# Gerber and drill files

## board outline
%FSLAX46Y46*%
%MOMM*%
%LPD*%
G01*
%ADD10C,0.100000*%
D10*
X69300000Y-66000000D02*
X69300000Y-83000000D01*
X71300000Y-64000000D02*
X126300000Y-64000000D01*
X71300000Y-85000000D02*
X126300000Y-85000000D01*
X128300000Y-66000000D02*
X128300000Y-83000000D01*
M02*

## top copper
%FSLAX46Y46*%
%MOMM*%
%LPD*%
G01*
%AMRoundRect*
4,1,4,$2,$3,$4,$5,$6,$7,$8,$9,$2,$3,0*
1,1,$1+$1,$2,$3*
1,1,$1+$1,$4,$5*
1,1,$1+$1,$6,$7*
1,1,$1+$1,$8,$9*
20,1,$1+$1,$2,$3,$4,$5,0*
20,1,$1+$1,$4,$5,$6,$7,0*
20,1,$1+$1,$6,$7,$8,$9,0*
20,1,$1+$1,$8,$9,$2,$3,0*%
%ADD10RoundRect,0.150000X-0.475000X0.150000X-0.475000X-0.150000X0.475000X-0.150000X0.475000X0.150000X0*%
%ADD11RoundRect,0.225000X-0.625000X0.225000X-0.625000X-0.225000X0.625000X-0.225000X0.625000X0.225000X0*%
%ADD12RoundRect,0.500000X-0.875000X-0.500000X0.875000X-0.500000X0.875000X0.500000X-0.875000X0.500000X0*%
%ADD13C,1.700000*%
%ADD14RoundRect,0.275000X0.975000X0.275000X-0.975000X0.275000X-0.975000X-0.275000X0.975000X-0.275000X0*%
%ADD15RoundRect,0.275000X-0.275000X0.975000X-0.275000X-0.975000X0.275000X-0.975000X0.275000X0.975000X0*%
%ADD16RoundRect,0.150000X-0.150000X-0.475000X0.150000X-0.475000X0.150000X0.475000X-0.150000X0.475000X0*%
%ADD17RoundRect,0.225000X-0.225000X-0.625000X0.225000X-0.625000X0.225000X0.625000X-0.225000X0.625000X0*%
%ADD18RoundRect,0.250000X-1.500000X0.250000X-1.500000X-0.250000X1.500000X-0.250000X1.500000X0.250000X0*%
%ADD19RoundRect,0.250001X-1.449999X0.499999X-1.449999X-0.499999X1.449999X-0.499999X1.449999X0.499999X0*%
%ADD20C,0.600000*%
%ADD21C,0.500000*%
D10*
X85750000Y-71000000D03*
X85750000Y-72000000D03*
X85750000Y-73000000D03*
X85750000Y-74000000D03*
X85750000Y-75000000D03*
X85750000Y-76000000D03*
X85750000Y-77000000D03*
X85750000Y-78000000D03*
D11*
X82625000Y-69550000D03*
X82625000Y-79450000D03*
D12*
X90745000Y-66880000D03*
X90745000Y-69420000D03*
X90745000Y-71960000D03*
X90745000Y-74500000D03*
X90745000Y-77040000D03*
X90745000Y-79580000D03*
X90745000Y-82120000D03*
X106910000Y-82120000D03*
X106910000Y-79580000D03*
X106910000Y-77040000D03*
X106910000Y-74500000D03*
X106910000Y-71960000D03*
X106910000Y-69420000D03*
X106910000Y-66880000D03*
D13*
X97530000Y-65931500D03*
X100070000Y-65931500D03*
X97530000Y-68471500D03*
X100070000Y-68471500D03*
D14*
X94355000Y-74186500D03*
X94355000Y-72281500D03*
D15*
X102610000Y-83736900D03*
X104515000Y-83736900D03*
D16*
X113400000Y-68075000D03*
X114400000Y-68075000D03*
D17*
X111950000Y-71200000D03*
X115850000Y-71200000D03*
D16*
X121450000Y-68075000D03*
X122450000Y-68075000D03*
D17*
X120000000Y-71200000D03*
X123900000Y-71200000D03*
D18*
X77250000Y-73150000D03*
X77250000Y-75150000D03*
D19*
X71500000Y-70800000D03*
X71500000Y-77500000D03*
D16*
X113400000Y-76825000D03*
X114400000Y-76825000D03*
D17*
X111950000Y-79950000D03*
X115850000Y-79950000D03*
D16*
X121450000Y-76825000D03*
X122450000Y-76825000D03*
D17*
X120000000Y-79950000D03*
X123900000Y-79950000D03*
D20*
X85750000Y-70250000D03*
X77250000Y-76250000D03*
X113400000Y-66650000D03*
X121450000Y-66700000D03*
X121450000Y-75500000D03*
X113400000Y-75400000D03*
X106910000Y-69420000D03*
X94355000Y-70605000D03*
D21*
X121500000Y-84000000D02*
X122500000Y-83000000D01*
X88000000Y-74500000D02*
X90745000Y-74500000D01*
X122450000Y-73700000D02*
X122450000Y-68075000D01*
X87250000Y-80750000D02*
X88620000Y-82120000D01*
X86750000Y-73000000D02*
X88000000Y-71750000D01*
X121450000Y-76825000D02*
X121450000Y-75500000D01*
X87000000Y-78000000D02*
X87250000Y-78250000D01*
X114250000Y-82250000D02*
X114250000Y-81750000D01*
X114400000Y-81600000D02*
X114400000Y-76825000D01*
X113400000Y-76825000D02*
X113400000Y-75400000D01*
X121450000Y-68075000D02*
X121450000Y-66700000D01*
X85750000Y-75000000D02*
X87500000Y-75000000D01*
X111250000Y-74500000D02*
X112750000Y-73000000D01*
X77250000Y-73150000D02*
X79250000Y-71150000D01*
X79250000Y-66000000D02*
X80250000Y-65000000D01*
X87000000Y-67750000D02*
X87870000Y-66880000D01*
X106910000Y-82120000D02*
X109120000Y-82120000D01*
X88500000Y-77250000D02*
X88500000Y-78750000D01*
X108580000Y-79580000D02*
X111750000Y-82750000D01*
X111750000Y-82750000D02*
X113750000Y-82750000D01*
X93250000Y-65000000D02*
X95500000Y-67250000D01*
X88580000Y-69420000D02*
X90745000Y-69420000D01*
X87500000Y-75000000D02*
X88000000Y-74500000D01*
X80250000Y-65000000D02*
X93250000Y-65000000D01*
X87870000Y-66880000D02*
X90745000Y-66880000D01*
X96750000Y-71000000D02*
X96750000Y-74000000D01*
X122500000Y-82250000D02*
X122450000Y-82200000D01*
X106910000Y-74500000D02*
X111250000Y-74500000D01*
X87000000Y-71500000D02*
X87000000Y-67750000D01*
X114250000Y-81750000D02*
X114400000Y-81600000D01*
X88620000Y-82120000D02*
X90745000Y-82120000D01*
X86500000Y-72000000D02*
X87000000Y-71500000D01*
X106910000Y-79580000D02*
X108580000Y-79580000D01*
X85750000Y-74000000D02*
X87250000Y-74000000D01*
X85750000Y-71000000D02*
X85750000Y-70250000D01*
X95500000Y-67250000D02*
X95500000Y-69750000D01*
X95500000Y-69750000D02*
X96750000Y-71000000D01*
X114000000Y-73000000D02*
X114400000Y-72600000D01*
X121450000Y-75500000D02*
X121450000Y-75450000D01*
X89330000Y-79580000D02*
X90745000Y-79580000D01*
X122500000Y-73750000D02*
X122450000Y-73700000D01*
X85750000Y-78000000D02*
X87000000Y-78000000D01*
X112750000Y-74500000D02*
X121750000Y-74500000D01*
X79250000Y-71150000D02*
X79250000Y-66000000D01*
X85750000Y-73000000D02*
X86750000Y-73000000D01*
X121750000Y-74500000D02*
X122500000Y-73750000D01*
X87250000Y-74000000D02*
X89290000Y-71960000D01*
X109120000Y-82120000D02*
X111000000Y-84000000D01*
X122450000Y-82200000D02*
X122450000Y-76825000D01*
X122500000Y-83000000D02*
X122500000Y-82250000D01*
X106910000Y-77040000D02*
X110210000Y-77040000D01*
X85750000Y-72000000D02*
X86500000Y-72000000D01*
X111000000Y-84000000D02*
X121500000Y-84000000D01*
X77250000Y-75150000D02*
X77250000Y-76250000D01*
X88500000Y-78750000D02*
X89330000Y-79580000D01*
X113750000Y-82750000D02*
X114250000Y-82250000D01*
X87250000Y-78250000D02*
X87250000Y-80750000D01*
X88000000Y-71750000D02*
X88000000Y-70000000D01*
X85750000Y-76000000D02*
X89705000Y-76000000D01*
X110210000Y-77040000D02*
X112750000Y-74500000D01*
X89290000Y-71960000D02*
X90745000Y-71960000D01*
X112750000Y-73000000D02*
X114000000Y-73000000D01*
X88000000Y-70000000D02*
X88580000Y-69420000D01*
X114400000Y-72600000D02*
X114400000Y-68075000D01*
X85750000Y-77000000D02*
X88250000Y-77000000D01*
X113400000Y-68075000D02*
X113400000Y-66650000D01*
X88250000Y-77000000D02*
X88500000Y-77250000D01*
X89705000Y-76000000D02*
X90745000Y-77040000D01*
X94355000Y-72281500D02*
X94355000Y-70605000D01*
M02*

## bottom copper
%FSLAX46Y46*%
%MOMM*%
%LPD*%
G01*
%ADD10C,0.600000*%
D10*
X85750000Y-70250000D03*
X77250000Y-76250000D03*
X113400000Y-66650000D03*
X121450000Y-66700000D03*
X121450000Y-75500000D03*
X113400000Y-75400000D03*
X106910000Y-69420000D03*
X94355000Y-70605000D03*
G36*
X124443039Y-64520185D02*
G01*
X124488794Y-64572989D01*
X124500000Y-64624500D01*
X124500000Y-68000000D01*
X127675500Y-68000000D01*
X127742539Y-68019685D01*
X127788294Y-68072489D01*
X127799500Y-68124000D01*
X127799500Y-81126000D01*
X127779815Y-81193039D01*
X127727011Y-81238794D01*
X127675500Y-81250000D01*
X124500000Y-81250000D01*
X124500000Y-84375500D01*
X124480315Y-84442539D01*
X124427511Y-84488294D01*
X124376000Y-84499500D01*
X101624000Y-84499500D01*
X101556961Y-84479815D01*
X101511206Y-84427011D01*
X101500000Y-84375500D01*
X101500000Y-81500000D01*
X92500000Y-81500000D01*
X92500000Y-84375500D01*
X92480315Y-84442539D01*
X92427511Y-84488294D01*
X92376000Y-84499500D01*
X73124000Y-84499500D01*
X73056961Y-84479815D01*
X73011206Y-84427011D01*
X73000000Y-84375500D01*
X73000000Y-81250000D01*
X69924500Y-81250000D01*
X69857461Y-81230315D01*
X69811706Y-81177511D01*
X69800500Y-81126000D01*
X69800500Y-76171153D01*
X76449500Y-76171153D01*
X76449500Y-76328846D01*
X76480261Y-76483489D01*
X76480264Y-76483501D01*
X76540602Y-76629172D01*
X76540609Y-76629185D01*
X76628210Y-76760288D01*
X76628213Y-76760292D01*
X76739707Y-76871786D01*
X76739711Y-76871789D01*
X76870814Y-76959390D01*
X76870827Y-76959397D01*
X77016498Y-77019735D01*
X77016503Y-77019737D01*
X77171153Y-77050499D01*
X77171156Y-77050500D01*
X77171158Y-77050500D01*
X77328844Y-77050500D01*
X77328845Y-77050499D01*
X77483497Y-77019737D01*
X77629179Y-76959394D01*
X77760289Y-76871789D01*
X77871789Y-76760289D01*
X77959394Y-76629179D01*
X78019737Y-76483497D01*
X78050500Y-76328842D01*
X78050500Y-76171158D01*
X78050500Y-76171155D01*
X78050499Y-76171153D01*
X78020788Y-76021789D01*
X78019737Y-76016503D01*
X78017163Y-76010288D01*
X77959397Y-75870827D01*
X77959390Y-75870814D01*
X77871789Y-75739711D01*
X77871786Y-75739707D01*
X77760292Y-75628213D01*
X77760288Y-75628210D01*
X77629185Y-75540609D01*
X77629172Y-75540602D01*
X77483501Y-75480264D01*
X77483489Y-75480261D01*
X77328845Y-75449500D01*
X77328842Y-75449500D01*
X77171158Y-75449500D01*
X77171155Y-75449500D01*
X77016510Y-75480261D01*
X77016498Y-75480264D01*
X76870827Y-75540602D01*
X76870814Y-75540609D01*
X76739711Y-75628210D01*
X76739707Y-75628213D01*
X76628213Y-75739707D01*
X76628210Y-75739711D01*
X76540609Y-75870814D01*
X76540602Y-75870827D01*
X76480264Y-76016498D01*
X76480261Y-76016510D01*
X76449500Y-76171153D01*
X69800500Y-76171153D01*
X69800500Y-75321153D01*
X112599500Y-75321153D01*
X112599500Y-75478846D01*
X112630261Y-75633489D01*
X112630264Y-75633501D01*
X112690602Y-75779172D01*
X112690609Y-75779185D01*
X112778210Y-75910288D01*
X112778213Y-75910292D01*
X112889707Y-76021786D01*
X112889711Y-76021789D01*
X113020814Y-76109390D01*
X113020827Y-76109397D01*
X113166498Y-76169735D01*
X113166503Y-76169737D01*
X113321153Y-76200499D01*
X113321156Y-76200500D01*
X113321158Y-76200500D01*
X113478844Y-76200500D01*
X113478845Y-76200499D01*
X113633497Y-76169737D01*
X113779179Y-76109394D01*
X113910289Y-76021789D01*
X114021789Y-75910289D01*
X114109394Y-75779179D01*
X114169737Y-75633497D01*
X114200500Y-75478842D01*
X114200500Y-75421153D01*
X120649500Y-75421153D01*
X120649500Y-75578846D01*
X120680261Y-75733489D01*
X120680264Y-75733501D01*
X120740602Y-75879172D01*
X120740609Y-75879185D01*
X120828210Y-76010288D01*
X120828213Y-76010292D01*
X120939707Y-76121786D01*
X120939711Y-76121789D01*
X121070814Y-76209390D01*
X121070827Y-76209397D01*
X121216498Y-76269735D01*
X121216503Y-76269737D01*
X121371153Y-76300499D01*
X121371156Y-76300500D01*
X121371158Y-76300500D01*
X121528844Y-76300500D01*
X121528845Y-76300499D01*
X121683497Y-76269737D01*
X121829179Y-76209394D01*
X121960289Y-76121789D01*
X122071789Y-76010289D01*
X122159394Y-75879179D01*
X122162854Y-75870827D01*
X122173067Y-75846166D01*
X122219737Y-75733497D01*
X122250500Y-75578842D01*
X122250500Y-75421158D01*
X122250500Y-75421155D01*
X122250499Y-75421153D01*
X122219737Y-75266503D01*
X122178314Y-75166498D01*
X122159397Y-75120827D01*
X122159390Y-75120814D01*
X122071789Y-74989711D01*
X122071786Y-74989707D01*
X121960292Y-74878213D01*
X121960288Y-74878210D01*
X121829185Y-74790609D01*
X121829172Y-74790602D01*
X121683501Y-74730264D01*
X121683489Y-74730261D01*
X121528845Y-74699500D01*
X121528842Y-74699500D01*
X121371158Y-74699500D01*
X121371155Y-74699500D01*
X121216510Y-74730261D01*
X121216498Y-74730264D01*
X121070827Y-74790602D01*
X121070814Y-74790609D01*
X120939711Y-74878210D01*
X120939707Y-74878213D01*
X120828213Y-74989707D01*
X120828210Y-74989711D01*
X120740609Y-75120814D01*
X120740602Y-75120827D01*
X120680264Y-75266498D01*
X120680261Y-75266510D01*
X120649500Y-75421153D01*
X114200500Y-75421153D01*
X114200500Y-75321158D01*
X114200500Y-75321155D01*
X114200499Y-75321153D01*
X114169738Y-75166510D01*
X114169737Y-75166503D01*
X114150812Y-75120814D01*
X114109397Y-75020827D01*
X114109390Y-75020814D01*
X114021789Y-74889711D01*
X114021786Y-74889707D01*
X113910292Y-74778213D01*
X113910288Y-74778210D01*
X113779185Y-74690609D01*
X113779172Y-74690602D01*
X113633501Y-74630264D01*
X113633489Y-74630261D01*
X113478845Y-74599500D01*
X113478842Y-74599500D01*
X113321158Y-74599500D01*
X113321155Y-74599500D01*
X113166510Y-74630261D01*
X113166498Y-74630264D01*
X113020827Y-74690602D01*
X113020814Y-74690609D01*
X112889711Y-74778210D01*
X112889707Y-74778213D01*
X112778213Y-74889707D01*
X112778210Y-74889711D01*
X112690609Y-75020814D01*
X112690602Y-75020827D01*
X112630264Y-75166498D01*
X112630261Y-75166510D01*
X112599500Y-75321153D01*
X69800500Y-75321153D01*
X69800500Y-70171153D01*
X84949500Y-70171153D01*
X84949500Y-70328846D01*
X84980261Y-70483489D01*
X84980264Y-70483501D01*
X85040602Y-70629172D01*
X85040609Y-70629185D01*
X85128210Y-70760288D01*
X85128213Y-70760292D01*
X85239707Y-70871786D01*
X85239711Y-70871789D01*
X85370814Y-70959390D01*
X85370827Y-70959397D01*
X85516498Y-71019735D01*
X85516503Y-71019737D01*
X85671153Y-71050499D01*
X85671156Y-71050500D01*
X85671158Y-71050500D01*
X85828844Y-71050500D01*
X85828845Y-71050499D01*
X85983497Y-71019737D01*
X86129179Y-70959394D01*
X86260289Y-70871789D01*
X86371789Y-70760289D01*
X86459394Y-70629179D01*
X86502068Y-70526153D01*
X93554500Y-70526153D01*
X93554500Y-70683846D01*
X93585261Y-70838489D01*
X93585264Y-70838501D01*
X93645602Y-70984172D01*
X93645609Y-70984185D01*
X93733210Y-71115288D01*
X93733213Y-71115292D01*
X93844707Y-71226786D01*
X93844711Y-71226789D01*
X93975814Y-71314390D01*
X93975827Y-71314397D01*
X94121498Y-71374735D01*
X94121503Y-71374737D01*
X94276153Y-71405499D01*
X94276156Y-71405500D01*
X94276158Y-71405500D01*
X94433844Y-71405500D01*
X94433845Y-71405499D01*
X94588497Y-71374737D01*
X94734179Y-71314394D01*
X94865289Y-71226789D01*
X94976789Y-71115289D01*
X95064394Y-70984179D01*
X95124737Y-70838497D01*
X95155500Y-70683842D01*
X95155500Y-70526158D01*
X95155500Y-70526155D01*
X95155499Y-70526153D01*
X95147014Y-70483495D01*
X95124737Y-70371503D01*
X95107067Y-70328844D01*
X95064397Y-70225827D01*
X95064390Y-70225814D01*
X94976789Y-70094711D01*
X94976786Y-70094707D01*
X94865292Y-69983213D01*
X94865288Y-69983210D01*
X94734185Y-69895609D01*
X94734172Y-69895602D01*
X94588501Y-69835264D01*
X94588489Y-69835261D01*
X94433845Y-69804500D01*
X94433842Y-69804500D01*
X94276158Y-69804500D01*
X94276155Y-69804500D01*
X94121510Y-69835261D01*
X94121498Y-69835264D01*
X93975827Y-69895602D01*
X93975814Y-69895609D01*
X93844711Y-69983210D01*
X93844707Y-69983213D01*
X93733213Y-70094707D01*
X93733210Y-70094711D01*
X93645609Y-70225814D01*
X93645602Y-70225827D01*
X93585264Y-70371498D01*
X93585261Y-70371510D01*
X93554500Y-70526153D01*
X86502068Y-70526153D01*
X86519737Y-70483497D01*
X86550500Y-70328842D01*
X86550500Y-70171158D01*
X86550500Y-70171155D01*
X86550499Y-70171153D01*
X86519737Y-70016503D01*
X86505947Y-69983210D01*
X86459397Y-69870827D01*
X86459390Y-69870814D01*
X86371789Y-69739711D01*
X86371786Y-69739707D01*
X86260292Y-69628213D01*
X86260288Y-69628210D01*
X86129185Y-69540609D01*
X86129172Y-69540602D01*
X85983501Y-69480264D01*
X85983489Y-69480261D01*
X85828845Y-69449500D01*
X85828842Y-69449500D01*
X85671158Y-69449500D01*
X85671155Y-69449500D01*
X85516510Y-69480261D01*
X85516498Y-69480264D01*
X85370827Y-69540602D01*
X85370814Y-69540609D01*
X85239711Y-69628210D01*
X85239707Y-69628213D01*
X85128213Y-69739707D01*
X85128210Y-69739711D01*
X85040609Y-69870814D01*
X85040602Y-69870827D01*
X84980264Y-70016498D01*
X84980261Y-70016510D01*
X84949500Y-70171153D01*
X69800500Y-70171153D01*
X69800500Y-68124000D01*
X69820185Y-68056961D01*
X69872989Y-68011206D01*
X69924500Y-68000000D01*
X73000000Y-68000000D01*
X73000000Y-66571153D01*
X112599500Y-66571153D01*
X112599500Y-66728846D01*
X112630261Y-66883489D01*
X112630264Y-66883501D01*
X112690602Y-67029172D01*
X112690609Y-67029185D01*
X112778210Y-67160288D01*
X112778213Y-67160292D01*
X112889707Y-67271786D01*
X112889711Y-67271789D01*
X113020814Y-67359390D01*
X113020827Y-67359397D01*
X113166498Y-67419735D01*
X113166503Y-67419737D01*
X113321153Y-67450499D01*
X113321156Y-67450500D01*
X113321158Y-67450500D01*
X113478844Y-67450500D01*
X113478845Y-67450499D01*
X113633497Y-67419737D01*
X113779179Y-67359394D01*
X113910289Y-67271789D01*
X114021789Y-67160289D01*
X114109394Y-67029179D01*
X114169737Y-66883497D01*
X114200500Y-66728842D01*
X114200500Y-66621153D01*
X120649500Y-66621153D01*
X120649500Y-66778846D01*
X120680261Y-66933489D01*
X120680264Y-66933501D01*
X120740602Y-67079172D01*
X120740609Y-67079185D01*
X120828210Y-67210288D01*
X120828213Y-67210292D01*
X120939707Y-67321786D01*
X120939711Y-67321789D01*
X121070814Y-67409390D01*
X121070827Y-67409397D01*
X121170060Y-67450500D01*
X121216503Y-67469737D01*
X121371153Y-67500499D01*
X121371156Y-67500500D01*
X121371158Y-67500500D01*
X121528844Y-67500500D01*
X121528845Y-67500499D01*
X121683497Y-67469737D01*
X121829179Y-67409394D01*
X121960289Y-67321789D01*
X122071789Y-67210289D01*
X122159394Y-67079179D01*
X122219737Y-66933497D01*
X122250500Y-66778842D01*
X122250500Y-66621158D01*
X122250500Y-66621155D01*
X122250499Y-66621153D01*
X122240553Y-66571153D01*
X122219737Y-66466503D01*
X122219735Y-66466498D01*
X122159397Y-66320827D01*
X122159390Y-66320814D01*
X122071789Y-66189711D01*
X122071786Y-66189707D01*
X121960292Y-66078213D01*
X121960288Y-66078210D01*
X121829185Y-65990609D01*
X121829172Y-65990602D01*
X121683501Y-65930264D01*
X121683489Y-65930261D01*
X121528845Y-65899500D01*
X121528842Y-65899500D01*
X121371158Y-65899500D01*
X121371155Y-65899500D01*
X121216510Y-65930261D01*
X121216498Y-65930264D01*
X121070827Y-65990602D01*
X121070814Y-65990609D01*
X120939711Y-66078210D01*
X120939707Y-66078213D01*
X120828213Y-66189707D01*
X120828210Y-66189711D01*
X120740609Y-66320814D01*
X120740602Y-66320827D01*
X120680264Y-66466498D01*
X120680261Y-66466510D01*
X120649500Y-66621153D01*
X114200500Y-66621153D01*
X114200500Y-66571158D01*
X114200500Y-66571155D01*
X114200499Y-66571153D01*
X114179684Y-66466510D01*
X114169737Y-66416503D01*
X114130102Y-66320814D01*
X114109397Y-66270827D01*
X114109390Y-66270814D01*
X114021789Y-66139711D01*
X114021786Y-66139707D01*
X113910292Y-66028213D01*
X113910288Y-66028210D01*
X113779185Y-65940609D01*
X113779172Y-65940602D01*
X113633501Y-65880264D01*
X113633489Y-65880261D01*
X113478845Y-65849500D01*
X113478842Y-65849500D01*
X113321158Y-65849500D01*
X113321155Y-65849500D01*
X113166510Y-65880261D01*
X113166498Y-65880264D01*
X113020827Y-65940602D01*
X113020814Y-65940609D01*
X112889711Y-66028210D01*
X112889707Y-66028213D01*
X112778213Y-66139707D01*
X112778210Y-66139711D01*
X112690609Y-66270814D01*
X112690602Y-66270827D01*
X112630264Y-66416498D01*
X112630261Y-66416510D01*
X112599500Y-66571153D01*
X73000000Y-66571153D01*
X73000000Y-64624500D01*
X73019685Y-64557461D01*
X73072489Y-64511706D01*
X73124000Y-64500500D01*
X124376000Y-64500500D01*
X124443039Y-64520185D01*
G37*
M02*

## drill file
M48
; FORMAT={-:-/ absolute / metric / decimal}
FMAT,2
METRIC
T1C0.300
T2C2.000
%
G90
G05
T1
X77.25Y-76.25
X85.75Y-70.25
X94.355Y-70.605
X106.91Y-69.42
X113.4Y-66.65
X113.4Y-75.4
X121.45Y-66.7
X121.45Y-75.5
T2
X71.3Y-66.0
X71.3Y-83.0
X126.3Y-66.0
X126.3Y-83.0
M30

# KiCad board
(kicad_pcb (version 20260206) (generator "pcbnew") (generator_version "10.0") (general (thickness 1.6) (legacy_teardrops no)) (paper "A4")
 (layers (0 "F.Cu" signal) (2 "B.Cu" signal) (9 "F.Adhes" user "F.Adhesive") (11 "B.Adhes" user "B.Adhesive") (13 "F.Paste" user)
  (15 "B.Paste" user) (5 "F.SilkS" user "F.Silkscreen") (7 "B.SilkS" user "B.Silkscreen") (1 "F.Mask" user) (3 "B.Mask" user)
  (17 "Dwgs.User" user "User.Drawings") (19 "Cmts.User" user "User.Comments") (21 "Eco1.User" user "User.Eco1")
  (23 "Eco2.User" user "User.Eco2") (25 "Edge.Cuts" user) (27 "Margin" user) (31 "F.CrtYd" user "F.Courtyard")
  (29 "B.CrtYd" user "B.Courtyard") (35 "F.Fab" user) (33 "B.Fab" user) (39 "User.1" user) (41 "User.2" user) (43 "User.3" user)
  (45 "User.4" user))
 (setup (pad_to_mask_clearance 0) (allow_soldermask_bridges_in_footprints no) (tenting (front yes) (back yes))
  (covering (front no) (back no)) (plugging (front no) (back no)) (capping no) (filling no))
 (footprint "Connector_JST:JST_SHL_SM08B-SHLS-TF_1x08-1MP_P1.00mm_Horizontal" (layer "F.Cu") (at 84.075 74.5 -90)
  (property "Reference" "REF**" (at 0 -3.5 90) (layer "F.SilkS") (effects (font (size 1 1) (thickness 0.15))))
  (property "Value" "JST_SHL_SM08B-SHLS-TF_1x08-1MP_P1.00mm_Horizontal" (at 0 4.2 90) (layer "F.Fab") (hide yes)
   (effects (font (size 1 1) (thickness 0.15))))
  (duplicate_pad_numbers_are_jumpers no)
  (pad "1" smd roundrect (at -3.5 -1.675 270) (size 0.6 1.25) (layers "F.Cu" "F.Mask" "F.Paste") (roundrect_rratio 0.25))
  (pad "2" smd roundrect (at -2.5 -1.675 270) (size 0.6 1.25) (layers "F.Cu" "F.Mask" "F.Paste") (roundrect_rratio 0.25))
  (pad "3" smd roundrect (at -1.5 -1.675 270) (size 0.6 1.25) (layers "F.Cu" "F.Mask" "F.Paste") (roundrect_rratio 0.25))
  (pad "4" smd roundrect (at -0.5 -1.675 270) (size 0.6 1.25) (layers "F.Cu" "F.Mask" "F.Paste") (roundrect_rratio 0.25))
  (pad "5" smd roundrect (at 0.5 -1.675 270) (size 0.6 1.25) (layers "F.Cu" "F.Mask" "F.Paste") (roundrect_rratio 0.25))
  (pad "6" smd roundrect (at 1.5 -1.675 270) (size 0.6 1.25) (layers "F.Cu" "F.Mask" "F.Paste") (roundrect_rratio 0.25))
  (pad "7" smd roundrect (at 2.5 -1.675 270) (size 0.6 1.25) (layers "F.Cu" "F.Mask" "F.Paste") (roundrect_rratio 0.25))
  (pad "8" smd roundrect (at 3.5 -1.675 270) (size 0.6 1.25) (layers "F.Cu" "F.Mask" "F.Paste") (roundrect_rratio 0.25))
  (pad "MP" smd roundrect (at -4.95 1.45 270) (size 0.9 1.7) (layers "F.Cu" "F.Mask" "F.Paste") (roundrect_rratio 0.25))
  (pad "MP" smd roundrect (at 4.95 1.45 270) (size 0.9 1.7) (layers "F.Cu" "F.Mask" "F.Paste") (roundrect_rratio 0.25)))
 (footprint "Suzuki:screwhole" (layer "F.Cu") (at 126.300001 65.999999)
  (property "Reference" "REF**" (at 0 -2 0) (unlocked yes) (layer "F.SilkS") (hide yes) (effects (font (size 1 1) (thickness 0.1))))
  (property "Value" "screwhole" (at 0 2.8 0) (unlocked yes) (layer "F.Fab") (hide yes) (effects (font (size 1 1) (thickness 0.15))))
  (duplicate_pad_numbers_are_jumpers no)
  (pad "" np_thru_hole circle (at 0 0) (size 2 2) (drill 2) (layers "*.Cu" "*.Mask")))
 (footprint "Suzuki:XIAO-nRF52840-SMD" (layer "F.Cu") (at 89.91 85)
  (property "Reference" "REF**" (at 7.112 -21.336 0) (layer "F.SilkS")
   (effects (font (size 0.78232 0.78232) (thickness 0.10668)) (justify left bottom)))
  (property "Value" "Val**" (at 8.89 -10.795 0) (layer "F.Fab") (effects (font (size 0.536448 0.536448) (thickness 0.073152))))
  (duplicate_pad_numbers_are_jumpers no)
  (pad "1" smd roundrect (at 0.835 -18.12) (size 2.75 2) (layers "F.Cu" "F.Mask" "F.Paste") (roundrect_rratio 0.25)
   (solder_mask_margin 0.0508) (thermal_bridge_angle 45))
  (pad "2" smd roundrect (at 0.835 -15.58) (size 2.75 2) (layers "F.Cu" "F.Mask" "F.Paste") (roundrect_rratio 0.25)
   (solder_mask_margin 0.0508) (thermal_bridge_angle 45))
  (pad "3" smd roundrect (at 0.835 -13.04) (size 2.75 2) (layers "F.Cu" "F.Mask" "F.Paste") (roundrect_rratio 0.25)
   (solder_mask_margin 0.0508) (thermal_bridge_angle 45))
  (pad "4" smd roundrect (at 0.835 -10.5) (size 2.75 2) (layers "F.Cu" "F.Mask" "F.Paste") (roundrect_rratio 0.25)
   (solder_mask_margin 0.0508) (thermal_bridge_angle 45))
  (pad "5" smd roundrect (at 0.835 -7.96) (size 2.75 2) (layers "F.Cu" "F.Mask" "F.Paste") (roundrect_rratio 0.25)
   (solder_mask_margin 0.0508) (thermal_bridge_angle 45))
  (pad "6" smd roundrect (at 0.835 -5.42) (size 2.75 2) (layers "F.Cu" "F.Mask" "F.Paste") (roundrect_rratio 0.25)
   (solder_mask_margin 0.0508) (thermal_bridge_angle 45))
  (pad "7" smd roundrect (at 0.835 -2.88) (size 2.75 2) (layers "F.Cu" "F.Mask" "F.Paste") (roundrect_rratio 0.25)
   (solder_mask_margin 0.0508) (thermal_bridge_angle 45))
  (pad "8" smd roundrect (at 17 -2.88) (size 2.75 2) (layers "F.Cu" "F.Mask" "F.Paste") (roundrect_rratio 0.25) (solder_mask_margin 0.0508)
   (thermal_bridge_angle 45))
  (pad "9" smd roundrect (at 17 -5.42) (size 2.75 2) (layers "F.Cu" "F.Mask" "F.Paste") (roundrect_rratio 0.25) (solder_mask_margin 0.0508)
   (thermal_bridge_angle 45))
  (pad "10" smd roundrect (at 17 -7.96) (size 2.75 2) (layers "F.Cu" "F.Mask" "F.Paste") (roundrect_rratio 0.25) (solder_mask_margin 0.0508)
   (thermal_bridge_angle 45))
  (pad "11" smd roundrect (at 17 -10.5) (size 2.75 2) (layers "F.Cu" "F.Mask" "F.Paste") (roundrect_rratio 0.25) (solder_mask_margin 0.0508)
   (thermal_bridge_angle 45))
  (pad "12" smd roundrect (at 17 -13.04) (size 2.75 2) (layers "F.Cu" "F.Mask" "F.Paste") (roundrect_rratio 0.25)
   (solder_mask_margin 0.0508) (thermal_bridge_angle 45))
  (pad "13" smd roundrect (at 17 -15.58) (size 2.75 2) (layers "F.Cu" "F.Mask" "F.Paste") (roundrect_rratio 0.25) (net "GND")
   (solder_mask_margin 0.0508) (thermal_bridge_angle 45))
  (pad "14" smd roundrect (at 17 -18.12) (size 2.75 2) (layers "F.Cu" "F.Mask" "F.Paste") (roundrect_rratio 0.25)
   (solder_mask_margin 0.0508) (thermal_bridge_angle 45))
  (pad "15" smd circle (at 7.62 -19.0685) (size 1.7 1.7) (layers "F.Cu" "F.Mask" "F.Paste"))
  (pad "16" smd circle (at 10.16 -19.0685) (size 1.7 1.7) (layers "F.Cu" "F.Mask" "F.Paste"))
  (pad "17" smd circle (at 7.62 -16.5285) (size 1.7 1.7) (layers "F.Cu" "F.Mask" "F.Paste"))
  (pad "18" smd circle (at 10.16 -16.5285) (size 1.7 1.7) (layers "F.Cu" "F.Mask" "F.Paste"))
  (pad "19" smd roundrect (at 4.445 -10.8135 180) (size 2.5 1.1) (layers "F.Cu" "F.Mask" "F.Paste") (roundrect_rratio 0.25) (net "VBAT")
   (thermal_bridge_angle 45))
  (pad "20" smd roundrect (at 4.445 -12.7185 180) (size 2.5 1.1) (layers "F.Cu" "F.Mask" "F.Paste") (roundrect_rratio 0.25) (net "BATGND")
   (thermal_bridge_angle 45))
  (pad "21" smd roundrect (at 12.7 -1.2631 270) (size 2.5 1.1) (layers "F.Cu" "F.Mask" "F.Paste") (roundrect_rratio 0.25)
   (thermal_bridge_angle 45))
  (pad "22" smd roundrect (at 14.605 -1.2631 270) (size 2.5 1.1) (layers "F.Cu" "F.Mask" "F.Paste") (roundrect_rratio 0.25)
   (thermal_bridge_angle 45)))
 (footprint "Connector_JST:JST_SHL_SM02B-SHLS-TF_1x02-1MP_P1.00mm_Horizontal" (layer "F.Cu") (at 113.9 69.75)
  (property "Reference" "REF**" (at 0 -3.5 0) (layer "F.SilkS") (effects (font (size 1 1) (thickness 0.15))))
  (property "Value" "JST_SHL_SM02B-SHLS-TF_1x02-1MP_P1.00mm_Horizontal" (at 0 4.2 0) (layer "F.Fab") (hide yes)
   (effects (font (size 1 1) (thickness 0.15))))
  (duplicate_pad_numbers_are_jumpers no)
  (pad "1" smd roundrect (at -0.5 -1.675) (size 0.6 1.25) (layers "F.Cu" "F.Mask" "F.Paste") (roundrect_rratio 0.25))
  (pad "2" smd roundrect (at 0.5 -1.675) (size 0.6 1.25) (layers "F.Cu" "F.Mask" "F.Paste") (roundrect_rratio 0.25))
  (pad "MP" smd roundrect (at -1.95 1.45) (size 0.9 1.7) (layers "F.Cu" "F.Mask" "F.Paste") (roundrect_rratio 0.25))
  (pad "MP" smd roundrect (at 1.95 1.45) (size 0.9 1.7) (layers "F.Cu" "F.Mask" "F.Paste") (roundrect_rratio 0.25)))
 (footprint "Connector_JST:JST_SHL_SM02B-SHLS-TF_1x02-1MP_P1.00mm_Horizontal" (layer "F.Cu") (at 121.95 69.75)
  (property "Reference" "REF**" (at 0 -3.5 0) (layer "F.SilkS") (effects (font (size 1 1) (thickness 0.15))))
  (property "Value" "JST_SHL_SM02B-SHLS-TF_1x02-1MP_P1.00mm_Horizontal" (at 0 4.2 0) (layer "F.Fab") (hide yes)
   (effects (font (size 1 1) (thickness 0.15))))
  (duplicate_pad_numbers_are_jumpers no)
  (pad "1" smd roundrect (at -0.5 -1.675) (size 0.6 1.25) (layers "F.Cu" "F.Mask" "F.Paste") (roundrect_rratio 0.25))
  (pad "2" smd roundrect (at 0.5 -1.675) (size 0.6 1.25) (layers "F.Cu" "F.Mask" "F.Paste") (roundrect_rratio 0.25))
  (pad "MP" smd roundrect (at -1.95 1.45) (size 0.9 1.7) (layers "F.Cu" "F.Mask" "F.Paste") (roundrect_rratio 0.25))
  (pad "MP" smd roundrect (at 1.95 1.45) (size 0.9 1.7) (layers "F.Cu" "F.Mask" "F.Paste") (roundrect_rratio 0.25)))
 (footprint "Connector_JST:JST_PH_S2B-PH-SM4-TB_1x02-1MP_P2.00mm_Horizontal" (layer "F.Cu") (at 74.4 74.15 -90)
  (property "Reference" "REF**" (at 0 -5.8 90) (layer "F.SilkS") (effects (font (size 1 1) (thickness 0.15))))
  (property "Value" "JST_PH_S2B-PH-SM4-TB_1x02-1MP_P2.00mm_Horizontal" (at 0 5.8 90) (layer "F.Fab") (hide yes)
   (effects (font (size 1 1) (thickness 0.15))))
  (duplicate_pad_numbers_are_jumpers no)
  (pad "1" smd roundrect (at -1 -2.85 270) (size 1 3.5) (layers "F.Cu" "F.Mask" "F.Paste") (roundrect_rratio 0.25))
  (pad "2" smd roundrect (at 1 -2.85 270) (size 1 3.5) (layers "F.Cu" "F.Mask" "F.Paste") (roundrect_rratio 0.25))
  (pad "MP" smd roundrect (at -3.35 2.9 270) (size 1.5 3.4) (layers "F.Cu" "F.Mask" "F.Paste") (roundrect_rratio 0.166667))
  (pad "MP" smd roundrect (at 3.35 2.9 270) (size 1.5 3.4) (layers "F.Cu" "F.Mask" "F.Paste") (roundrect_rratio 0.166667)))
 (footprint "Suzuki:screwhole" (layer "F.Cu") (at 71.299999 83.000001)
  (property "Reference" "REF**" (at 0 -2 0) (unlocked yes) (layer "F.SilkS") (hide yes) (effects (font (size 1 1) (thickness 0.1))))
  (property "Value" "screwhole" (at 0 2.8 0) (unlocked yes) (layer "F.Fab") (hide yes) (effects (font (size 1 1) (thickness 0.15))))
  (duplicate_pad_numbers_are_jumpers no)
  (pad "" np_thru_hole circle (at 0 0) (size 2 2) (drill 2) (layers "*.Cu" "*.Mask")))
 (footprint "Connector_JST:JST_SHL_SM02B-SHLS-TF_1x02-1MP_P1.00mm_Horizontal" (layer "F.Cu") (at 113.9 78.5)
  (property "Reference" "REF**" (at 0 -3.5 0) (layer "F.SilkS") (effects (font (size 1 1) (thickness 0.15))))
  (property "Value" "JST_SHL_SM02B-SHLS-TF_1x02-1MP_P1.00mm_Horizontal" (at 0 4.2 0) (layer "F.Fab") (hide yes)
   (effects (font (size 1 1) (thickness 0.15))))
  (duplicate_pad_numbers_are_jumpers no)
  (pad "1" smd roundrect (at -0.5 -1.675) (size 0.6 1.25) (layers "F.Cu" "F.Mask" "F.Paste") (roundrect_rratio 0.25))
  (pad "2" smd roundrect (at 0.5 -1.675) (size 0.6 1.25) (layers "F.Cu" "F.Mask" "F.Paste") (roundrect_rratio 0.25))
  (pad "MP" smd roundrect (at -1.95 1.45) (size 0.9 1.7) (layers "F.Cu" "F.Mask" "F.Paste") (roundrect_rratio 0.25))
  (pad "MP" smd roundrect (at 1.95 1.45) (size 0.9 1.7) (layers "F.Cu" "F.Mask" "F.Paste") (roundrect_rratio 0.25)))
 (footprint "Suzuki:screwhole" (layer "F.Cu") (at 126.300001 83.000001)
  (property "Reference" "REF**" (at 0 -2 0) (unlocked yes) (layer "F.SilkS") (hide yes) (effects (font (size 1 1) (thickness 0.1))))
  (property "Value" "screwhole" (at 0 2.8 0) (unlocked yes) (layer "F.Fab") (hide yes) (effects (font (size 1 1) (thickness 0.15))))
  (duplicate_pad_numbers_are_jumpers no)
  (pad "" np_thru_hole circle (at 0 0) (size 2 2) (drill 2) (layers "*.Cu" "*.Mask")))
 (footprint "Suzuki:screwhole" (layer "F.Cu") (at 71.299999 65.999999)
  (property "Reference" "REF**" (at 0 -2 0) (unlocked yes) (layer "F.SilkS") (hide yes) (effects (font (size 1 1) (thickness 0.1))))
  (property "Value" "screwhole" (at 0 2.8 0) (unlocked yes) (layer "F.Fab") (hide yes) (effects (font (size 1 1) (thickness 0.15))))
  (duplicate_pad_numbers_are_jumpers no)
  (pad "" np_thru_hole circle (at 0 0) (size 2 2) (drill 2) (layers "*.Cu" "*.Mask")))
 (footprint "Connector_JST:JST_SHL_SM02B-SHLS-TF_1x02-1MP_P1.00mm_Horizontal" (layer "F.Cu") (at 121.95 78.5)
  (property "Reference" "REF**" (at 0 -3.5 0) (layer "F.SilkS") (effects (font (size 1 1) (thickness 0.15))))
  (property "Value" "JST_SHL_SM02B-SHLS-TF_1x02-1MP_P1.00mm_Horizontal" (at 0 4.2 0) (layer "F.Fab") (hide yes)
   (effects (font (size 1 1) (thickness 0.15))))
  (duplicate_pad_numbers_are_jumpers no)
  (pad "1" smd roundrect (at -0.5 -1.675) (size 0.6 1.25) (layers "F.Cu" "F.Mask" "F.Paste") (roundrect_rratio 0.25))
  (pad "2" smd roundrect (at 0.5 -1.675) (size 0.6 1.25) (layers "F.Cu" "F.Mask" "F.Paste") (roundrect_rratio 0.25))
  (pad "MP" smd roundrect (at -1.95 1.45) (size 0.9 1.7) (layers "F.Cu" "F.Mask" "F.Paste") (roundrect_rratio 0.25))
  (pad "MP" smd roundrect (at 1.95 1.45) (size 0.9 1.7) (layers "F.Cu" "F.Mask" "F.Paste") (roundrect_rratio 0.25)))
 (gr_line (start 69.3 66) (end 69.3 83) (stroke (width 0.1) (type solid)) (layer "Edge.Cuts"))
 (gr_line (start 71.3 64) (end 126.3 64) (stroke (width 0.1) (type solid)) (layer "Edge.Cuts"))
 (gr_line (start 71.3 85) (end 126.3 85) (stroke (width 0.1) (type solid)) (layer "Edge.Cuts"))
 (gr_line (start 128.3 66) (end 128.3 83) (stroke (width 0.1) (type solid)) (layer "Edge.Cuts"))
 (segment (start 121.5 84) (end 122.5 83) (width 0.5) (layer "F.Cu") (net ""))
 (segment (start 88 74.5) (end 90.745 74.5) (width 0.5) (layer "F.Cu") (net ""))
 (segment (start 122.45 73.7) (end 122.45 68.075) (width 0.5) (layer "F.Cu") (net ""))
 (segment (start 87.25 80.75) (end 88.62 82.12) (width 0.5) (layer "F.Cu") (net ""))
 (segment (start 86.75 73) (end 88 71.75) (width 0.5) (layer "F.Cu") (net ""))
 (segment (start 121.45 76.825) (end 121.45 75.5) (width 0.5) (layer "F.Cu") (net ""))
 (segment (start 87 78) (end 87.25 78.25) (width 0.5) (layer "F.Cu") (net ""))
 (segment (start 114.25 82.25) (end 114.25 81.75) (width 0.5) (layer "F.Cu") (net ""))
 (segment (start 114.4 81.6) (end 114.4 76.825) (width 0.5) (layer "F.Cu") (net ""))
 (segment (start 113.4 76.825) (end 113.4 75.4) (width 0.5) (layer "F.Cu") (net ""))
 (segment (start 121.45 68.075) (end 121.45 66.7) (width 0.5) (layer "F.Cu") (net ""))
 (segment (start 85.75 75) (end 87.5 75) (width 0.5) (layer "F.Cu") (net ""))
 (segment (start 111.25 74.5) (end 112.75 73) (width 0.5) (layer "F.Cu") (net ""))
 (segment (start 77.25 73.15) (end 79.25 71.15) (width 0.5) (layer "F.Cu") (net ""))
 (segment (start 79.25 66) (end 80.25 65) (width 0.5) (layer "F.Cu") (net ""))
 (segment (start 87 67.75) (end 87.87 66.88) (width 0.5) (layer "F.Cu") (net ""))
 (segment (start 106.91 82.12) (end 109.12 82.12) (width 0.5) (layer "F.Cu") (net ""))
 (segment (start 88.5 77.25) (end 88.5 78.75) (width 0.5) (layer "F.Cu") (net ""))
 (segment (start 108.58 79.58) (end 111.75 82.75) (width 0.5) (layer "F.Cu") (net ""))
 (segment (start 111.75 82.75) (end 113.75 82.75) (width 0.5) (layer "F.Cu") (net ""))
 (segment (start 93.25 65) (end 95.5 67.25) (width 0.5) (layer "F.Cu") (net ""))
 (segment (start 88.58 69.42) (end 90.745 69.42) (width 0.5) (layer "F.Cu") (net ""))
 (segment (start 87.5 75) (end 88 74.5) (width 0.5) (layer "F.Cu") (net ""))
 (segment (start 80.25 65) (end 93.25 65) (width 0.5) (layer "F.Cu") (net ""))
 (segment (start 87.87 66.88) (end 90.745 66.88) (width 0.5) (layer "F.Cu") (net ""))
 (segment (start 96.75 71) (end 96.75 74) (width 0.5) (layer "F.Cu") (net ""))
 (segment (start 122.5 82.25) (end 122.45 82.2) (width 0.5) (layer "F.Cu") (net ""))
 (segment (start 106.91 74.5) (end 111.25 74.5) (width 0.5) (layer "F.Cu") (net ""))
 (segment (start 87 71.5) (end 87 67.75) (width 0.5) (layer "F.Cu") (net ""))
 (segment (start 114.25 81.75) (end 114.4 81.6) (width 0.5) (layer "F.Cu") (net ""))
 (segment (start 88.62 82.12) (end 90.745 82.12) (width 0.5) (layer "F.Cu") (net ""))
 (segment (start 86.5 72) (end 87 71.5) (width 0.5) (layer "F.Cu") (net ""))
 (segment (start 106.91 79.58) (end 108.58 79.58) (width 0.5) (layer "F.Cu") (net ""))
 (segment (start 85.75 74) (end 87.25 74) (width 0.5) (layer "F.Cu") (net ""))
 (segment (start 85.75 71) (end 85.75 70.25) (width 0.5) (layer "F.Cu") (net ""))
 (segment (start 95.5 67.25) (end 95.5 69.75) (width 0.5) (layer "F.Cu") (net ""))
 (segment (start 95.5 69.75) (end 96.75 71) (width 0.5) (layer "F.Cu") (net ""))
 (segment (start 114 73) (end 114.4 72.6) (width 0.5) (layer "F.Cu") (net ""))
 (segment (start 121.45 75.5) (end 121.45 75.45) (width 0.5) (layer "F.Cu") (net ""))
 (segment (start 89.33 79.58) (end 90.745 79.58) (width 0.5) (layer "F.Cu") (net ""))
 (segment (start 122.5 73.75) (end 122.45 73.7) (width 0.5) (layer "F.Cu") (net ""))
 (segment (start 85.75 78) (end 87 78) (width 0.5) (layer "F.Cu") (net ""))
 (segment (start 112.75 74.5) (end 121.75 74.5) (width 0.5) (layer "F.Cu") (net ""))
 (segment (start 79.25 71.15) (end 79.25 66) (width 0.5) (layer "F.Cu") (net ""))
 (segment (start 85.75 73) (end 86.75 73) (width 0.5) (layer "F.Cu") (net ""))
 (segment (start 121.75 74.5) (end 122.5 73.75) (width 0.5) (layer "F.Cu") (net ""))
 (segment (start 87.25 74) (end 89.29 71.96) (width 0.5) (layer "F.Cu") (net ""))
 (segment (start 109.12 82.12) (end 111 84) (width 0.5) (layer "F.Cu") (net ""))
 (segment (start 122.45 82.2) (end 122.45 76.825) (width 0.5) (layer "F.Cu") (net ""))
 (segment (start 122.5 83) (end 122.5 82.25) (width 0.5) (layer "F.Cu") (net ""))
 (segment (start 106.91 77.04) (end 110.21 77.04) (width 0.5) (layer "F.Cu") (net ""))
 (segment (start 85.75 72) (end 86.5 72) (width 0.5) (layer "F.Cu") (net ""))
 (segment (start 111 84) (end 121.5 84) (width 0.5) (layer "F.Cu") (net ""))
 (segment (start 77.25 75.15) (end 77.25 76.25) (width 0.5) (layer "F.Cu") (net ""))
 (segment (start 88.5 78.75) (end 89.33 79.58) (width 0.5) (layer "F.Cu") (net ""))
 (segment (start 113.75 82.75) (end 114.25 82.25) (width 0.5) (layer "F.Cu") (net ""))
 (segment (start 87.25 78.25) (end 87.25 80.75) (width 0.5) (layer "F.Cu") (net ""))
 (segment (start 88 71.75) (end 88 70) (width 0.5) (layer "F.Cu") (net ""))
 (segment (start 85.75 76) (end 89.705 76) (width 0.5) (layer "F.Cu") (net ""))
 (segment (start 110.21 77.04) (end 112.75 74.5) (width 0.5) (layer "F.Cu") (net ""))
 (segment (start 89.29 71.96) (end 90.745 71.96) (width 0.5) (layer "F.Cu") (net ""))
 (segment (start 112.75 73) (end 114 73) (width 0.5) (layer "F.Cu") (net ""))
 (segment (start 88 70) (end 88.58 69.42) (width 0.5) (layer "F.Cu") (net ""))
 (segment (start 114.4 72.6) (end 114.4 68.075) (width 0.5) (layer "F.Cu") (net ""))
 (segment (start 85.75 77) (end 88.25 77) (width 0.5) (layer "F.Cu") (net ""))
 (segment (start 113.4 68.075) (end 113.4 66.65) (width 0.5) (layer "F.Cu") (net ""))
 (segment (start 88.25 77) (end 88.5 77.25) (width 0.5) (layer "F.Cu") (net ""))
 (segment (start 89.705 76) (end 90.745 77.04) (width 0.5) (layer "F.Cu") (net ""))
 (via (at 85.75 70.25) (size 0.6) (drill 0.3) (layers "F.Cu" "B.Cu") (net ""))
 (via (at 77.25 76.25) (size 0.6) (drill 0.3) (layers "F.Cu" "B.Cu") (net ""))
 (via (at 113.4 66.65) (size 0.6) (drill 0.3) (layers "F.Cu" "B.Cu") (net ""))
 (via (at 121.45 66.7) (size 0.6) (drill 0.3) (layers "F.Cu" "B.Cu") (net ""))
 (via (at 121.45 75.5) (size 0.6) (drill 0.3) (layers "F.Cu" "B.Cu") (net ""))
 (via (at 113.4 75.4) (size 0.6) (drill 0.3) (layers "F.Cu" "B.Cu") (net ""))
 (via (at 106.91 69.42) (size 0.6) (drill 0.3) (layers "F.Cu" "B.Cu") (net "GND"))
 (segment (start 94.355 72.2815) (end 94.355 70.605) (width 0.5) (layer "F.Cu") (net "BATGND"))
 (via (at 94.355 70.605) (size 0.6) (drill 0.3) (layers "F.Cu" "B.Cu") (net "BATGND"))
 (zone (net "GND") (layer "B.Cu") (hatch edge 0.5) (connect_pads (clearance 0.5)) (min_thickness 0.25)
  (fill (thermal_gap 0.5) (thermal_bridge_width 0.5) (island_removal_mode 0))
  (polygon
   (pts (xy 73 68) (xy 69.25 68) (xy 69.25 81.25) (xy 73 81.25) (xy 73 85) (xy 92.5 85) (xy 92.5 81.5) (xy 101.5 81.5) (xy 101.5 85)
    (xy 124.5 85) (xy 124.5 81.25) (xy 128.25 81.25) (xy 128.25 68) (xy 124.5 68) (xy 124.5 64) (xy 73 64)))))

